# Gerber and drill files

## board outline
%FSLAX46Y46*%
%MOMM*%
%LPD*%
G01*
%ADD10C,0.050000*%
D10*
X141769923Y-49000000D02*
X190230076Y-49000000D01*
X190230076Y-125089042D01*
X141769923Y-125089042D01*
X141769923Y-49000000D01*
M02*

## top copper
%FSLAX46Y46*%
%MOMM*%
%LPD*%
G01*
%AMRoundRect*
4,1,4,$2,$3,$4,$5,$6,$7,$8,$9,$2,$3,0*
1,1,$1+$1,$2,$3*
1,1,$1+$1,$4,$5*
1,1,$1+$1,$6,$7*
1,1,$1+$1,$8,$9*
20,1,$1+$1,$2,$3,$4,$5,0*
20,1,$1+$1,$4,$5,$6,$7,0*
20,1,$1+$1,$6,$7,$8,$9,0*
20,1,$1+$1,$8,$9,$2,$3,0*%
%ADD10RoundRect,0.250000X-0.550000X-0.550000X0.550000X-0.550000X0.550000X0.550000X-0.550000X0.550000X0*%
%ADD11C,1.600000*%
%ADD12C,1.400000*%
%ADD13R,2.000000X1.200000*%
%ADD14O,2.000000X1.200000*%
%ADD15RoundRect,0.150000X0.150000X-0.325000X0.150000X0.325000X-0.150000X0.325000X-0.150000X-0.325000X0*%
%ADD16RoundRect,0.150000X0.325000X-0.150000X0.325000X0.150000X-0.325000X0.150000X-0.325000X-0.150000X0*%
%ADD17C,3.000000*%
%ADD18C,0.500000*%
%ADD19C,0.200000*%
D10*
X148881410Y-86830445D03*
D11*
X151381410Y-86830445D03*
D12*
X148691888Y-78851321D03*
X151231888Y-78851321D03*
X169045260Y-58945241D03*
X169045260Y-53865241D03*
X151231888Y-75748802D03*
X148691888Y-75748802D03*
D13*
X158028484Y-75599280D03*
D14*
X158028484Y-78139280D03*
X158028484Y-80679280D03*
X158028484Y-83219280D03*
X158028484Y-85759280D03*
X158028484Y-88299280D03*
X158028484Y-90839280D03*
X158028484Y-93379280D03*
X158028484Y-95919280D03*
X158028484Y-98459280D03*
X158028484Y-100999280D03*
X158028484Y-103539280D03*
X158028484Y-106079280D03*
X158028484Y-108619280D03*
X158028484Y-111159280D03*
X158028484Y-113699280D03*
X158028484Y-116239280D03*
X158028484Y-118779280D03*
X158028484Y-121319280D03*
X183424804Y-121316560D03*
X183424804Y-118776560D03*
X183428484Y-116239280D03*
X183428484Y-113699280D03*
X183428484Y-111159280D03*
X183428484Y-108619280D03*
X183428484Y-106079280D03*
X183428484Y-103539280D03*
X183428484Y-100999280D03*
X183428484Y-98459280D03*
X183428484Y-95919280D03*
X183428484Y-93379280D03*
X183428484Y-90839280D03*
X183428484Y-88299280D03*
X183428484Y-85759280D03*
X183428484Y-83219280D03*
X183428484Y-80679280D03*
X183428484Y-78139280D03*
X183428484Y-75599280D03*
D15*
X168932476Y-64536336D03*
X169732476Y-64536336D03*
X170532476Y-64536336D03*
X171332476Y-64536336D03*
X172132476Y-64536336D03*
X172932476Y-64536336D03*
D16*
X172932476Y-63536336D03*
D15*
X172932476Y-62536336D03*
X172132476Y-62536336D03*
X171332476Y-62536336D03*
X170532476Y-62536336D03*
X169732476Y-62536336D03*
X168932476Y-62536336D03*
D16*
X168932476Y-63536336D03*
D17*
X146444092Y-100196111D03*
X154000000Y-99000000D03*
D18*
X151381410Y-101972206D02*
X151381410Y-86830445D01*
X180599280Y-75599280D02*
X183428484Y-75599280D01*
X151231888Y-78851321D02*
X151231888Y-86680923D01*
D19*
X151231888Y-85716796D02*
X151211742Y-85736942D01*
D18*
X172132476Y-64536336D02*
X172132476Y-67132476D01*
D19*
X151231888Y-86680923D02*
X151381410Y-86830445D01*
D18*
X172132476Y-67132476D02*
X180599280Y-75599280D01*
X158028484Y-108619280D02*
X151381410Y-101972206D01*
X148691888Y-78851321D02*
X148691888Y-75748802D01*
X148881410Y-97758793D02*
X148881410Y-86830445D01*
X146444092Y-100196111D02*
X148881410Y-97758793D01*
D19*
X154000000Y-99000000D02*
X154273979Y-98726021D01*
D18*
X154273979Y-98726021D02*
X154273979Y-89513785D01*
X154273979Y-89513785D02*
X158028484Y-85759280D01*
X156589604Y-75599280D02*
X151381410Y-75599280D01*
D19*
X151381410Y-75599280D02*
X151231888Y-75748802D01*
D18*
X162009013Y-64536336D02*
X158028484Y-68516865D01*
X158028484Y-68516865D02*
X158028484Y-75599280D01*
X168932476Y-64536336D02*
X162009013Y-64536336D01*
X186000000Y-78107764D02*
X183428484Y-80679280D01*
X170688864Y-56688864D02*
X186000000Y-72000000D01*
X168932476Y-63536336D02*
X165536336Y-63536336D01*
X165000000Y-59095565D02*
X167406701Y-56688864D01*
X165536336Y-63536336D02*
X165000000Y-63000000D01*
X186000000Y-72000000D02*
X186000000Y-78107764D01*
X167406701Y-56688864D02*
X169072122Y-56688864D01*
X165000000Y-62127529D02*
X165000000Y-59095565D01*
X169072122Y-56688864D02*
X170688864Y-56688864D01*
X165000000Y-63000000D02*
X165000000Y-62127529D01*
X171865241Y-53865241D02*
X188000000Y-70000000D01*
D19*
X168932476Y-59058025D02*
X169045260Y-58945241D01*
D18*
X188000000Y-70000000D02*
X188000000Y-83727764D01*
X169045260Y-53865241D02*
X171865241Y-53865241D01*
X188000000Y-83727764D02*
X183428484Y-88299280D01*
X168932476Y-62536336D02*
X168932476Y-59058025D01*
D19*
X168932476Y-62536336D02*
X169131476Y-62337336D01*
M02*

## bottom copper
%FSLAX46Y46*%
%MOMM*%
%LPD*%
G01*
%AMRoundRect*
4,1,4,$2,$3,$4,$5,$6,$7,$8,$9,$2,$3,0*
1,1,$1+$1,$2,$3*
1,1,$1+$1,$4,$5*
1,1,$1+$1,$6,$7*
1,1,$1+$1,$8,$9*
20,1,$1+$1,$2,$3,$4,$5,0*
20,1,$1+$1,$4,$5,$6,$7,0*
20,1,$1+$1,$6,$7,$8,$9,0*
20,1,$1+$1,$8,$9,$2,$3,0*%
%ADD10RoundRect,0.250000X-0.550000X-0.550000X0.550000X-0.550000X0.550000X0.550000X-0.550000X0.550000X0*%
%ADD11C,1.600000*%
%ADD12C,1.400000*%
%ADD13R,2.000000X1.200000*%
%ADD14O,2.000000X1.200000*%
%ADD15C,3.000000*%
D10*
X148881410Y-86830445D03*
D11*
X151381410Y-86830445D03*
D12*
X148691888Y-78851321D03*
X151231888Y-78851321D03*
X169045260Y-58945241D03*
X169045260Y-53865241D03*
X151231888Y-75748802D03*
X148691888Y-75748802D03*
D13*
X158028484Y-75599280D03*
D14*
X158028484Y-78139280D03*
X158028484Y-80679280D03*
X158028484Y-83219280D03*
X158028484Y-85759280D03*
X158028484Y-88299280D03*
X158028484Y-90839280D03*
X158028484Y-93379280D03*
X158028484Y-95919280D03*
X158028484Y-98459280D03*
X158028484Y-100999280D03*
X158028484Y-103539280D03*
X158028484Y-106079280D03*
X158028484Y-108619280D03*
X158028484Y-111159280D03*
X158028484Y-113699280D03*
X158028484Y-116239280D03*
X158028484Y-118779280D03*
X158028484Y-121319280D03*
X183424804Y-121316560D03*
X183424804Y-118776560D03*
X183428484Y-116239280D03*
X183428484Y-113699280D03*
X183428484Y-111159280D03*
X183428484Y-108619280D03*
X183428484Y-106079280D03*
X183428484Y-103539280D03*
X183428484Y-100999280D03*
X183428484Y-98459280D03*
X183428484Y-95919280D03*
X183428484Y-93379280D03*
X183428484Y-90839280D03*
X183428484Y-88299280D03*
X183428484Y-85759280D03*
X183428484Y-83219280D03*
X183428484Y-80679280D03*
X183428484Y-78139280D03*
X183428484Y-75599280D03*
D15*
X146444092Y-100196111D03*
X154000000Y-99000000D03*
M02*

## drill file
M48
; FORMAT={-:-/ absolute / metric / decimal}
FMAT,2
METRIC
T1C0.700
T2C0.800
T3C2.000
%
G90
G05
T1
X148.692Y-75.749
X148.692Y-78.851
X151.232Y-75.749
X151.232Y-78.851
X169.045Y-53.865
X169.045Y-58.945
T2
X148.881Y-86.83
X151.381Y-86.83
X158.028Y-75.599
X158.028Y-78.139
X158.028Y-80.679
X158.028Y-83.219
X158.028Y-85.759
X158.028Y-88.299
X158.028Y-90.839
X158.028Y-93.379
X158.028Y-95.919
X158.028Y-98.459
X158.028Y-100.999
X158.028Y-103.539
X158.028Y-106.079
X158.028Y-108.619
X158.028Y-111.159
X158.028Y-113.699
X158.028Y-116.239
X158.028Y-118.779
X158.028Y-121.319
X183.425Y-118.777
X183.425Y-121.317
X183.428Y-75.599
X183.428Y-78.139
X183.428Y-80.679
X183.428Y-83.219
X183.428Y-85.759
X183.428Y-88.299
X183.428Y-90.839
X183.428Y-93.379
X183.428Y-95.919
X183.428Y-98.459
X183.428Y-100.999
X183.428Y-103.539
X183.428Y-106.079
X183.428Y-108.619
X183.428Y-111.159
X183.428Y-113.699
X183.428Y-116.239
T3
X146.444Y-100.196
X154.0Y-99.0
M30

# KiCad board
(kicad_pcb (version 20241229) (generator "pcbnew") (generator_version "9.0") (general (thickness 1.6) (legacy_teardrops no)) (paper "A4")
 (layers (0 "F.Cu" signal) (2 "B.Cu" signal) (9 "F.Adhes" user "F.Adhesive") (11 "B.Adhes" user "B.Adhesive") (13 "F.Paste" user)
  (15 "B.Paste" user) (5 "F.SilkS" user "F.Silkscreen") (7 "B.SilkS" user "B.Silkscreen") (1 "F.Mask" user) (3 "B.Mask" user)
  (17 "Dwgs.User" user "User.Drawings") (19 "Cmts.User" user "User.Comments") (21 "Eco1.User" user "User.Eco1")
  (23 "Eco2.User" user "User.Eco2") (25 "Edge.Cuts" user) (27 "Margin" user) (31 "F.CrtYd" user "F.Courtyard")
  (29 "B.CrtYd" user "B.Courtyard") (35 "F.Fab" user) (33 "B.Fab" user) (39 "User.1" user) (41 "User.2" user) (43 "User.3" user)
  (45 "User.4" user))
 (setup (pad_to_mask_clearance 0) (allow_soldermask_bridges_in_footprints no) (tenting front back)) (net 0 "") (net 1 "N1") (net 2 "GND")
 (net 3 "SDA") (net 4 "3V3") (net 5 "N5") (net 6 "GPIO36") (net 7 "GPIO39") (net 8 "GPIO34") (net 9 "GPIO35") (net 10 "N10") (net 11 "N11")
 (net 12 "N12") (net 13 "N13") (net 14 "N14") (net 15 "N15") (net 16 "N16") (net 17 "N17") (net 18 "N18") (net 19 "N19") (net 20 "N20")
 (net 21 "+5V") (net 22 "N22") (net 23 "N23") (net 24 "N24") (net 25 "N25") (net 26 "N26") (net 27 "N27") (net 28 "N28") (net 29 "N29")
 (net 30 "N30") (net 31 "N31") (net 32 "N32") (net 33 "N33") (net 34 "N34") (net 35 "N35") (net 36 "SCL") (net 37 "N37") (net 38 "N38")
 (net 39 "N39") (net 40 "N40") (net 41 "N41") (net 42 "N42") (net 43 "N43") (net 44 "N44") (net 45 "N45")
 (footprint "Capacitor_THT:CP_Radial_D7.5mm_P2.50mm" (layer "F.Cu") (at 148.88141 86.830445)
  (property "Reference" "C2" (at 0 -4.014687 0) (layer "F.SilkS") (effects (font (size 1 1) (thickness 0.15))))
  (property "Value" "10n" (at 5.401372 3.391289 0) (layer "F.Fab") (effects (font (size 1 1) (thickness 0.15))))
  (pad "1" thru_hole roundrect (at 0 0) (size 1.6 1.6) (drill 0.8) (layers "*.Cu" "*.Mask") (remove_unused_layers no)
   (roundrect_rratio 0.15625) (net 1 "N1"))
  (pad "2" thru_hole circle (at 2.5 0) (size 1.6 1.6) (drill 0.8) (layers "*.Cu" "*.Mask") (remove_unused_layers no) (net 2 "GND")))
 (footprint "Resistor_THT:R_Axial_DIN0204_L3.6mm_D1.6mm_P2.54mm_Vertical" (layer "F.Cu") (at 148.691888 78.851321)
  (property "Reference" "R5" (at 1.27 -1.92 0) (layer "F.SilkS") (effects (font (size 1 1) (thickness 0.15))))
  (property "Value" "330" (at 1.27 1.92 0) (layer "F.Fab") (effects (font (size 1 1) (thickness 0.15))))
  (pad "1" thru_hole circle (at 0 0) (size 1.4 1.4) (drill 0.7) (layers "*.Cu" "*.Mask") (remove_unused_layers no) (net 1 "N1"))
  (pad "2" thru_hole circle (at 2.54 0) (size 1.4 1.4) (drill 0.7) (layers "*.Cu" "*.Mask") (remove_unused_layers no) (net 2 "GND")))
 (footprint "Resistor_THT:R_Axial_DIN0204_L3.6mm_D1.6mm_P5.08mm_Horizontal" (layer "F.Cu") (at 169.04526 58.945241 90)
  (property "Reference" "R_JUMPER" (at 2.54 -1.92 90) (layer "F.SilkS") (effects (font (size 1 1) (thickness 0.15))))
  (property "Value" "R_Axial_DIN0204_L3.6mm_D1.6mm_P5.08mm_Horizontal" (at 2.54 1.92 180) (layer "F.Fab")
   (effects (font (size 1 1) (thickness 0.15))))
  (pad "1" thru_hole circle (at 0 0 90) (size 1.4 1.4) (drill 0.7) (layers "*.Cu" "*.Mask") (remove_unused_layers no) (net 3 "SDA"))
  (pad "2" thru_hole circle (at 5.08 0 90) (size 1.4 1.4) (drill 0.7) (layers "*.Cu" "*.Mask") (remove_unused_layers no) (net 3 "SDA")))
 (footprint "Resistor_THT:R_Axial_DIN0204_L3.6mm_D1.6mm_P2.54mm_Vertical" (layer "F.Cu") (at 151.231888 75.748802 180)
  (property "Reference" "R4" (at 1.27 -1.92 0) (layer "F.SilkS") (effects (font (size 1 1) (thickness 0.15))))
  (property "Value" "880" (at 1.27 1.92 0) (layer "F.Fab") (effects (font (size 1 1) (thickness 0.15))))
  (pad "1" thru_hole circle (at 0 0 180) (size 1.4 1.4) (drill 0.7) (layers "*.Cu" "*.Mask") (remove_unused_layers no) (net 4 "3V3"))
  (pad "2" thru_hole circle (at 2.54 0 180) (size 1.4 1.4) (drill 0.7) (layers "*.Cu" "*.Mask") (remove_unused_layers no) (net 1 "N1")))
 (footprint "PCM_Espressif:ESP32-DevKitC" (layer "F.Cu") (at 158.028484 75.59928)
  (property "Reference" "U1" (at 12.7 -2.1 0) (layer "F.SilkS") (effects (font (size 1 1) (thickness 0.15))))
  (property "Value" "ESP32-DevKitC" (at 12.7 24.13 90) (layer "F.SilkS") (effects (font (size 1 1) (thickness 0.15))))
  (pad "1" thru_hole rect (at 0 0 270) (size 1.2 2) (drill 0.8) (layers "*.Cu" "*.Mask") (remove_unused_layers no) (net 4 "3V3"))
  (pad "2" thru_hole oval (at 0 2.54 270) (size 1.2 2) (drill 0.8) (layers "*.Cu" "*.Mask") (remove_unused_layers no) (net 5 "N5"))
  (pad "3" thru_hole oval (at 0 5.08 270) (size 1.2 2) (drill 0.8) (layers "*.Cu" "*.Mask") (remove_unused_layers no) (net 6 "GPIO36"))
  (pad "4" thru_hole oval (at 0 7.62 270) (size 1.2 2) (drill 0.8) (layers "*.Cu" "*.Mask") (remove_unused_layers no) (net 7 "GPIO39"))
  (pad "5" thru_hole oval (at 0 10.16 270) (size 1.2 2) (drill 0.8) (layers "*.Cu" "*.Mask") (remove_unused_layers no) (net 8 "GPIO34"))
  (pad "6" thru_hole oval (at 0 12.7 270) (size 1.2 2) (drill 0.8) (layers "*.Cu" "*.Mask") (remove_unused_layers no) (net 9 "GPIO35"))
  (pad "7" thru_hole oval (at 0 15.24 270) (size 1.2 2) (drill 0.8) (layers "*.Cu" "*.Mask") (remove_unused_layers no) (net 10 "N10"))
  (pad "8" thru_hole oval (at 0 17.78 270) (size 1.2 2) (drill 0.8) (layers "*.Cu" "*.Mask") (remove_unused_layers no) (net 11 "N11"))
  (pad "9" thru_hole oval (at 0 20.32 270) (size 1.2 2) (drill 0.8) (layers "*.Cu" "*.Mask") (remove_unused_layers no) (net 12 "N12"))
  (pad "10" thru_hole oval (at 0 22.86 270) (size 1.2 2) (drill 0.8) (layers "*.Cu" "*.Mask") (remove_unused_layers no) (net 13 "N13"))
  (pad "11" thru_hole oval (at 0 25.4 270) (size 1.2 2) (drill 0.8) (layers "*.Cu" "*.Mask") (remove_unused_layers no) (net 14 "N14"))
  (pad "12" thru_hole oval (at 0 27.94 270) (size 1.2 2) (drill 0.8) (layers "*.Cu" "*.Mask") (remove_unused_layers no) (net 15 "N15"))
  (pad "13" thru_hole oval (at 0 30.48 270) (size 1.2 2) (drill 0.8) (layers "*.Cu" "*.Mask") (remove_unused_layers no) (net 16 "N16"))
  (pad "14" thru_hole oval (at 0 33.02 270) (size 1.2 2) (drill 0.8) (layers "*.Cu" "*.Mask") (remove_unused_layers no) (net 2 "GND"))
  (pad "15" thru_hole oval (at 0 35.56 270) (size 1.2 2) (drill 0.8) (layers "*.Cu" "*.Mask") (remove_unused_layers no) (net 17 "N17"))
  (pad "16" thru_hole oval (at 0 38.1 270) (size 1.2 2) (drill 0.8) (layers "*.Cu" "*.Mask") (remove_unused_layers no) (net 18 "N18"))
  (pad "17" thru_hole oval (at 0 40.64 270) (size 1.2 2) (drill 0.8) (layers "*.Cu" "*.Mask") (remove_unused_layers no) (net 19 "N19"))
  (pad "18" thru_hole oval (at 0 43.18 270) (size 1.2 2) (drill 0.8) (layers "*.Cu" "*.Mask") (remove_unused_layers no) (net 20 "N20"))
  (pad "19" thru_hole oval (at 0 45.72 270) (size 1.2 2) (drill 0.8) (layers "*.Cu" "*.Mask") (remove_unused_layers no) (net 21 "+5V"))
  (pad "20" thru_hole oval (at 25.39632 45.71728 270) (size 1.2 2) (drill 0.8) (layers "*.Cu" "*.Mask") (remove_unused_layers no)
   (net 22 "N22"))
  (pad "21" thru_hole oval (at 25.39632 43.17728 270) (size 1.2 2) (drill 0.8) (layers "*.Cu" "*.Mask") (remove_unused_layers no)
   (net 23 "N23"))
  (pad "22" thru_hole oval (at 25.4 40.64 270) (size 1.2 2) (drill 0.8) (layers "*.Cu" "*.Mask") (remove_unused_layers no) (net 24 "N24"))
  (pad "23" thru_hole oval (at 25.4 38.1 270) (size 1.2 2) (drill 0.8) (layers "*.Cu" "*.Mask") (remove_unused_layers no) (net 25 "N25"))
  (pad "24" thru_hole oval (at 25.4 35.56 270) (size 1.2 2) (drill 0.8) (layers "*.Cu" "*.Mask") (remove_unused_layers no) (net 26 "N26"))
  (pad "25" thru_hole oval (at 25.4 33.02 270) (size 1.2 2) (drill 0.8) (layers "*.Cu" "*.Mask") (remove_unused_layers no) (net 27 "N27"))
  (pad "26" thru_hole oval (at 25.4 30.48 270) (size 1.2 2) (drill 0.8) (layers "*.Cu" "*.Mask") (remove_unused_layers no) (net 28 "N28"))
  (pad "27" thru_hole oval (at 25.4 27.94 270) (size 1.2 2) (drill 0.8) (layers "*.Cu" "*.Mask") (remove_unused_layers no) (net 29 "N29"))
  (pad "28" thru_hole oval (at 25.4 25.4 270) (size 1.2 2) (drill 0.8) (layers "*.Cu" "*.Mask") (remove_unused_layers no) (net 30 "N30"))
  (pad "29" thru_hole oval (at 25.4 22.86 270) (size 1.2 2) (drill 0.8) (layers "*.Cu" "*.Mask") (remove_unused_layers no) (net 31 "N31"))
  (pad "30" thru_hole oval (at 25.4 20.32 270) (size 1.2 2) (drill 0.8) (layers "*.Cu" "*.Mask") (remove_unused_layers no) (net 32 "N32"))
  (pad "31" thru_hole oval (at 25.4 17.78 270) (size 1.2 2) (drill 0.8) (layers "*.Cu" "*.Mask") (remove_unused_layers no) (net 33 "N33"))
  (pad "32" thru_hole oval (at 25.4 15.24 270) (size 1.2 2) (drill 0.8) (layers "*.Cu" "*.Mask") (remove_unused_layers no) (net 2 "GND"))
  (pad "33" thru_hole oval (at 25.4 12.7 270) (size 1.2 2) (drill 0.8) (layers "*.Cu" "*.Mask") (remove_unused_layers no) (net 3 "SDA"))
  (pad "34" thru_hole oval (at 25.4 10.16 270) (size 1.2 2) (drill 0.8) (layers "*.Cu" "*.Mask") (remove_unused_layers no) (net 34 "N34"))
  (pad "35" thru_hole oval (at 25.4 7.62 270) (size 1.2 2) (drill 0.8) (layers "*.Cu" "*.Mask") (remove_unused_layers no) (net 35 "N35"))
  (pad "36" thru_hole oval (at 25.4 5.08 270) (size 1.2 2) (drill 0.8) (layers "*.Cu" "*.Mask") (remove_unused_layers no) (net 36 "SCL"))
  (pad "37" thru_hole oval (at 25.4 2.54 270) (size 1.2 2) (drill 0.8) (layers "*.Cu" "*.Mask") (remove_unused_layers no) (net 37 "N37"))
  (pad "38" thru_hole oval (at 25.4 0 270) (size 1.2 2) (drill 0.8) (layers "*.Cu" "*.Mask") (remove_unused_layers no) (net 2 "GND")))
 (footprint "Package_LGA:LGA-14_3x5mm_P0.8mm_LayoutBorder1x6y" (layer "F.Cu") (at 170.932476 63.536336 90)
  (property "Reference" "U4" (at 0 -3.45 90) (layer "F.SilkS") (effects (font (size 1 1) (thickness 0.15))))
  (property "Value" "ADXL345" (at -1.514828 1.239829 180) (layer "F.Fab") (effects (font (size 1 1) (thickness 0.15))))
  (pad "1" smd roundrect (at -1 -2 90) (size 0.95 0.6) (layers "F.Cu" "F.Mask" "F.Paste") (roundrect_rratio 0.25) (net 4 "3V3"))
  (pad "2" smd roundrect (at -1 -1.2 90) (size 0.95 0.6) (layers "F.Cu" "F.Mask" "F.Paste") (roundrect_rratio 0.25) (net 2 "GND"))
  (pad "3" smd roundrect (at -1 -0.4 90) (size 0.95 0.6) (layers "F.Cu" "F.Mask" "F.Paste") (roundrect_rratio 0.25) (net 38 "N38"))
  (pad "4" smd roundrect (at -1 0.4 90) (size 0.95 0.6) (layers "F.Cu" "F.Mask" "F.Paste") (roundrect_rratio 0.25) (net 2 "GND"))
  (pad "5" smd roundrect (at -1 1.2 90) (size 0.95 0.6) (layers "F.Cu" "F.Mask" "F.Paste") (roundrect_rratio 0.25) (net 2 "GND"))
  (pad "6" smd roundrect (at -1 2 90) (size 0.95 0.6) (layers "F.Cu" "F.Mask" "F.Paste") (roundrect_rratio 0.25) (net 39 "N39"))
  (pad "7" smd roundrect (at 0 2 90) (size 0.6 0.95) (layers "F.Cu" "F.Mask" "F.Paste") (roundrect_rratio 0.25) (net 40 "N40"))
  (pad "8" smd roundrect (at 1 2 90) (size 0.95 0.6) (layers "F.Cu" "F.Mask" "F.Paste") (roundrect_rratio 0.25) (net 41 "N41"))
  (pad "9" smd roundrect (at 1 1.2 90) (size 0.95 0.6) (layers "F.Cu" "F.Mask" "F.Paste") (roundrect_rratio 0.25) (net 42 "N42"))
  (pad "10" smd roundrect (at 1 0.4 90) (size 0.95 0.6) (layers "F.Cu" "F.Mask" "F.Paste") (roundrect_rratio 0.25) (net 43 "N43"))
  (pad "11" smd roundrect (at 1 -0.4 90) (size 0.95 0.6) (layers "F.Cu" "F.Mask" "F.Paste") (roundrect_rratio 0.25) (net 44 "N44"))
  (pad "12" smd roundrect (at 1 -1.2 90) (size 0.95 0.6) (layers "F.Cu" "F.Mask" "F.Paste") (roundrect_rratio 0.25) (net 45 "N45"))
  (pad "13" smd roundrect (at 1 -2 90) (size 0.95 0.6) (layers "F.Cu" "F.Mask" "F.Paste") (roundrect_rratio 0.25) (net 3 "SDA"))
  (pad "14" smd roundrect (at 0 -2 90) (size 0.6 0.95) (layers "F.Cu" "F.Mask" "F.Paste") (roundrect_rratio 0.25) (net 36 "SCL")))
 (gr_rect (start 141.769923 49) (end 190.230076 125.089042) (stroke (width 0.05) (type default)) (fill no) (layer "Edge.Cuts"))
 (segment (start 151.38141 101.972206) (end 151.38141 86.830445) (width 0.5) (layer "F.Cu") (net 2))
 (segment (start 180.59928 75.59928) (end 183.428484 75.59928) (width 0.5) (layer "F.Cu") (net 2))
 (segment (start 151.231888 78.851321) (end 151.231888 86.680923) (width 0.5) (layer "F.Cu") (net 2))
 (segment (start 151.231888 85.716796) (end 151.211742 85.736942) (width 0.2) (layer "F.Cu") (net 2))
 (segment (start 172.132476 64.536336) (end 172.132476 67.132476) (width 0.5) (layer "F.Cu") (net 2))
 (segment (start 151.231888 86.680923) (end 151.38141 86.830445) (width 0.2) (layer "F.Cu") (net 2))
 (segment (start 172.132476 67.132476) (end 180.59928 75.59928) (width 0.5) (layer "F.Cu") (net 2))
 (segment (start 158.028484 108.61928) (end 151.38141 101.972206) (width 0.5) (layer "F.Cu") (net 2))
 (segment (start 148.691888 78.851321) (end 148.691888 75.748802) (width 0.5) (layer "F.Cu") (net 1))
 (segment (start 148.88141 97.758793) (end 148.88141 86.830445) (width 0.5) (layer "F.Cu") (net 1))
 (segment (start 146.444092 100.196111) (end 148.88141 97.758793) (width 0.5) (layer "F.Cu") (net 1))
 (via (at 146.444092 100.196111) (size 3) (drill 2) (layers "F.Cu" "B.Cu") (free yes) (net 1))
 (segment (start 154 99) (end 154.273979 98.726021) (width 0.2) (layer "F.Cu") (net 8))
 (segment (start 154.273979 98.726021) (end 154.273979 89.513785) (width 0.5) (layer "F.Cu") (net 8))
 (segment (start 154.273979 89.513785) (end 158.028484 85.75928) (width 0.5) (layer "F.Cu") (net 8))
 (via (at 154 99) (size 3) (drill 2) (layers "F.Cu" "B.Cu") (free yes) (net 8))
 (segment (start 156.589604 75.59928) (end 151.38141 75.59928) (width 0.5) (layer "F.Cu") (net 4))
 (segment (start 151.38141 75.59928) (end 151.231888 75.748802) (width 0.2) (layer "F.Cu") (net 4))
 (segment (start 162.009013 64.536336) (end 158.028484 68.516865) (width 0.5) (layer "F.Cu") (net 4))
 (segment (start 158.028484 68.516865) (end 158.028484 75.59928) (width 0.5) (layer "F.Cu") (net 4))
 (segment (start 168.932476 64.536336) (end 162.009013 64.536336) (width 0.5) (layer "F.Cu") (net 4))
 (segment (start 186 78.107764) (end 183.428484 80.67928) (width 0.5) (layer "F.Cu") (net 36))
 (segment (start 170.688864 56.688864) (end 186 72) (width 0.5) (layer "F.Cu") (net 36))
 (segment (start 168.932476 63.536336) (end 165.536336 63.536336) (width 0.5) (layer "F.Cu") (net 36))
 (segment (start 165 59.095565) (end 167.406701 56.688864) (width 0.5) (layer "F.Cu") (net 36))
 (segment (start 165.536336 63.536336) (end 165 63) (width 0.5) (layer "F.Cu") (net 36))
 (segment (start 186 72) (end 186 78.107764) (width 0.5) (layer "F.Cu") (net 36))
 (segment (start 167.406701 56.688864) (end 169.072122 56.688864) (width 0.5) (layer "F.Cu") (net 36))
 (segment (start 165 62.127529) (end 165 59.095565) (width 0.5) (layer "F.Cu") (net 36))
 (segment (start 169.072122 56.688864) (end 170.688864 56.688864) (width 0.5) (layer "F.Cu") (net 36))
 (segment (start 165 63) (end 165 62.127529) (width 0.5) (layer "F.Cu") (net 36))
 (segment (start 171.865241 53.865241) (end 188 70) (width 0.5) (layer "F.Cu") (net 3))
 (segment (start 168.932476 59.058025) (end 169.04526 58.945241) (width 0.2) (layer "F.Cu") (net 3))
 (segment (start 188 70) (end 188 83.727764) (width 0.5) (layer "F.Cu") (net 3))
 (segment (start 169.04526 53.865241) (end 171.865241 53.865241) (width 0.5) (layer "F.Cu") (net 3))
 (segment (start 188 83.727764) (end 183.428484 88.29928) (width 0.5) (layer "F.Cu") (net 3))
 (segment (start 168.932476 62.536336) (end 168.932476 59.058025) (width 0.5) (layer "F.Cu") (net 3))
 (segment (start 168.932476 62.536336) (end 169.131476 62.337336) (width 0.2) (layer "F.Cu") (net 3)))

